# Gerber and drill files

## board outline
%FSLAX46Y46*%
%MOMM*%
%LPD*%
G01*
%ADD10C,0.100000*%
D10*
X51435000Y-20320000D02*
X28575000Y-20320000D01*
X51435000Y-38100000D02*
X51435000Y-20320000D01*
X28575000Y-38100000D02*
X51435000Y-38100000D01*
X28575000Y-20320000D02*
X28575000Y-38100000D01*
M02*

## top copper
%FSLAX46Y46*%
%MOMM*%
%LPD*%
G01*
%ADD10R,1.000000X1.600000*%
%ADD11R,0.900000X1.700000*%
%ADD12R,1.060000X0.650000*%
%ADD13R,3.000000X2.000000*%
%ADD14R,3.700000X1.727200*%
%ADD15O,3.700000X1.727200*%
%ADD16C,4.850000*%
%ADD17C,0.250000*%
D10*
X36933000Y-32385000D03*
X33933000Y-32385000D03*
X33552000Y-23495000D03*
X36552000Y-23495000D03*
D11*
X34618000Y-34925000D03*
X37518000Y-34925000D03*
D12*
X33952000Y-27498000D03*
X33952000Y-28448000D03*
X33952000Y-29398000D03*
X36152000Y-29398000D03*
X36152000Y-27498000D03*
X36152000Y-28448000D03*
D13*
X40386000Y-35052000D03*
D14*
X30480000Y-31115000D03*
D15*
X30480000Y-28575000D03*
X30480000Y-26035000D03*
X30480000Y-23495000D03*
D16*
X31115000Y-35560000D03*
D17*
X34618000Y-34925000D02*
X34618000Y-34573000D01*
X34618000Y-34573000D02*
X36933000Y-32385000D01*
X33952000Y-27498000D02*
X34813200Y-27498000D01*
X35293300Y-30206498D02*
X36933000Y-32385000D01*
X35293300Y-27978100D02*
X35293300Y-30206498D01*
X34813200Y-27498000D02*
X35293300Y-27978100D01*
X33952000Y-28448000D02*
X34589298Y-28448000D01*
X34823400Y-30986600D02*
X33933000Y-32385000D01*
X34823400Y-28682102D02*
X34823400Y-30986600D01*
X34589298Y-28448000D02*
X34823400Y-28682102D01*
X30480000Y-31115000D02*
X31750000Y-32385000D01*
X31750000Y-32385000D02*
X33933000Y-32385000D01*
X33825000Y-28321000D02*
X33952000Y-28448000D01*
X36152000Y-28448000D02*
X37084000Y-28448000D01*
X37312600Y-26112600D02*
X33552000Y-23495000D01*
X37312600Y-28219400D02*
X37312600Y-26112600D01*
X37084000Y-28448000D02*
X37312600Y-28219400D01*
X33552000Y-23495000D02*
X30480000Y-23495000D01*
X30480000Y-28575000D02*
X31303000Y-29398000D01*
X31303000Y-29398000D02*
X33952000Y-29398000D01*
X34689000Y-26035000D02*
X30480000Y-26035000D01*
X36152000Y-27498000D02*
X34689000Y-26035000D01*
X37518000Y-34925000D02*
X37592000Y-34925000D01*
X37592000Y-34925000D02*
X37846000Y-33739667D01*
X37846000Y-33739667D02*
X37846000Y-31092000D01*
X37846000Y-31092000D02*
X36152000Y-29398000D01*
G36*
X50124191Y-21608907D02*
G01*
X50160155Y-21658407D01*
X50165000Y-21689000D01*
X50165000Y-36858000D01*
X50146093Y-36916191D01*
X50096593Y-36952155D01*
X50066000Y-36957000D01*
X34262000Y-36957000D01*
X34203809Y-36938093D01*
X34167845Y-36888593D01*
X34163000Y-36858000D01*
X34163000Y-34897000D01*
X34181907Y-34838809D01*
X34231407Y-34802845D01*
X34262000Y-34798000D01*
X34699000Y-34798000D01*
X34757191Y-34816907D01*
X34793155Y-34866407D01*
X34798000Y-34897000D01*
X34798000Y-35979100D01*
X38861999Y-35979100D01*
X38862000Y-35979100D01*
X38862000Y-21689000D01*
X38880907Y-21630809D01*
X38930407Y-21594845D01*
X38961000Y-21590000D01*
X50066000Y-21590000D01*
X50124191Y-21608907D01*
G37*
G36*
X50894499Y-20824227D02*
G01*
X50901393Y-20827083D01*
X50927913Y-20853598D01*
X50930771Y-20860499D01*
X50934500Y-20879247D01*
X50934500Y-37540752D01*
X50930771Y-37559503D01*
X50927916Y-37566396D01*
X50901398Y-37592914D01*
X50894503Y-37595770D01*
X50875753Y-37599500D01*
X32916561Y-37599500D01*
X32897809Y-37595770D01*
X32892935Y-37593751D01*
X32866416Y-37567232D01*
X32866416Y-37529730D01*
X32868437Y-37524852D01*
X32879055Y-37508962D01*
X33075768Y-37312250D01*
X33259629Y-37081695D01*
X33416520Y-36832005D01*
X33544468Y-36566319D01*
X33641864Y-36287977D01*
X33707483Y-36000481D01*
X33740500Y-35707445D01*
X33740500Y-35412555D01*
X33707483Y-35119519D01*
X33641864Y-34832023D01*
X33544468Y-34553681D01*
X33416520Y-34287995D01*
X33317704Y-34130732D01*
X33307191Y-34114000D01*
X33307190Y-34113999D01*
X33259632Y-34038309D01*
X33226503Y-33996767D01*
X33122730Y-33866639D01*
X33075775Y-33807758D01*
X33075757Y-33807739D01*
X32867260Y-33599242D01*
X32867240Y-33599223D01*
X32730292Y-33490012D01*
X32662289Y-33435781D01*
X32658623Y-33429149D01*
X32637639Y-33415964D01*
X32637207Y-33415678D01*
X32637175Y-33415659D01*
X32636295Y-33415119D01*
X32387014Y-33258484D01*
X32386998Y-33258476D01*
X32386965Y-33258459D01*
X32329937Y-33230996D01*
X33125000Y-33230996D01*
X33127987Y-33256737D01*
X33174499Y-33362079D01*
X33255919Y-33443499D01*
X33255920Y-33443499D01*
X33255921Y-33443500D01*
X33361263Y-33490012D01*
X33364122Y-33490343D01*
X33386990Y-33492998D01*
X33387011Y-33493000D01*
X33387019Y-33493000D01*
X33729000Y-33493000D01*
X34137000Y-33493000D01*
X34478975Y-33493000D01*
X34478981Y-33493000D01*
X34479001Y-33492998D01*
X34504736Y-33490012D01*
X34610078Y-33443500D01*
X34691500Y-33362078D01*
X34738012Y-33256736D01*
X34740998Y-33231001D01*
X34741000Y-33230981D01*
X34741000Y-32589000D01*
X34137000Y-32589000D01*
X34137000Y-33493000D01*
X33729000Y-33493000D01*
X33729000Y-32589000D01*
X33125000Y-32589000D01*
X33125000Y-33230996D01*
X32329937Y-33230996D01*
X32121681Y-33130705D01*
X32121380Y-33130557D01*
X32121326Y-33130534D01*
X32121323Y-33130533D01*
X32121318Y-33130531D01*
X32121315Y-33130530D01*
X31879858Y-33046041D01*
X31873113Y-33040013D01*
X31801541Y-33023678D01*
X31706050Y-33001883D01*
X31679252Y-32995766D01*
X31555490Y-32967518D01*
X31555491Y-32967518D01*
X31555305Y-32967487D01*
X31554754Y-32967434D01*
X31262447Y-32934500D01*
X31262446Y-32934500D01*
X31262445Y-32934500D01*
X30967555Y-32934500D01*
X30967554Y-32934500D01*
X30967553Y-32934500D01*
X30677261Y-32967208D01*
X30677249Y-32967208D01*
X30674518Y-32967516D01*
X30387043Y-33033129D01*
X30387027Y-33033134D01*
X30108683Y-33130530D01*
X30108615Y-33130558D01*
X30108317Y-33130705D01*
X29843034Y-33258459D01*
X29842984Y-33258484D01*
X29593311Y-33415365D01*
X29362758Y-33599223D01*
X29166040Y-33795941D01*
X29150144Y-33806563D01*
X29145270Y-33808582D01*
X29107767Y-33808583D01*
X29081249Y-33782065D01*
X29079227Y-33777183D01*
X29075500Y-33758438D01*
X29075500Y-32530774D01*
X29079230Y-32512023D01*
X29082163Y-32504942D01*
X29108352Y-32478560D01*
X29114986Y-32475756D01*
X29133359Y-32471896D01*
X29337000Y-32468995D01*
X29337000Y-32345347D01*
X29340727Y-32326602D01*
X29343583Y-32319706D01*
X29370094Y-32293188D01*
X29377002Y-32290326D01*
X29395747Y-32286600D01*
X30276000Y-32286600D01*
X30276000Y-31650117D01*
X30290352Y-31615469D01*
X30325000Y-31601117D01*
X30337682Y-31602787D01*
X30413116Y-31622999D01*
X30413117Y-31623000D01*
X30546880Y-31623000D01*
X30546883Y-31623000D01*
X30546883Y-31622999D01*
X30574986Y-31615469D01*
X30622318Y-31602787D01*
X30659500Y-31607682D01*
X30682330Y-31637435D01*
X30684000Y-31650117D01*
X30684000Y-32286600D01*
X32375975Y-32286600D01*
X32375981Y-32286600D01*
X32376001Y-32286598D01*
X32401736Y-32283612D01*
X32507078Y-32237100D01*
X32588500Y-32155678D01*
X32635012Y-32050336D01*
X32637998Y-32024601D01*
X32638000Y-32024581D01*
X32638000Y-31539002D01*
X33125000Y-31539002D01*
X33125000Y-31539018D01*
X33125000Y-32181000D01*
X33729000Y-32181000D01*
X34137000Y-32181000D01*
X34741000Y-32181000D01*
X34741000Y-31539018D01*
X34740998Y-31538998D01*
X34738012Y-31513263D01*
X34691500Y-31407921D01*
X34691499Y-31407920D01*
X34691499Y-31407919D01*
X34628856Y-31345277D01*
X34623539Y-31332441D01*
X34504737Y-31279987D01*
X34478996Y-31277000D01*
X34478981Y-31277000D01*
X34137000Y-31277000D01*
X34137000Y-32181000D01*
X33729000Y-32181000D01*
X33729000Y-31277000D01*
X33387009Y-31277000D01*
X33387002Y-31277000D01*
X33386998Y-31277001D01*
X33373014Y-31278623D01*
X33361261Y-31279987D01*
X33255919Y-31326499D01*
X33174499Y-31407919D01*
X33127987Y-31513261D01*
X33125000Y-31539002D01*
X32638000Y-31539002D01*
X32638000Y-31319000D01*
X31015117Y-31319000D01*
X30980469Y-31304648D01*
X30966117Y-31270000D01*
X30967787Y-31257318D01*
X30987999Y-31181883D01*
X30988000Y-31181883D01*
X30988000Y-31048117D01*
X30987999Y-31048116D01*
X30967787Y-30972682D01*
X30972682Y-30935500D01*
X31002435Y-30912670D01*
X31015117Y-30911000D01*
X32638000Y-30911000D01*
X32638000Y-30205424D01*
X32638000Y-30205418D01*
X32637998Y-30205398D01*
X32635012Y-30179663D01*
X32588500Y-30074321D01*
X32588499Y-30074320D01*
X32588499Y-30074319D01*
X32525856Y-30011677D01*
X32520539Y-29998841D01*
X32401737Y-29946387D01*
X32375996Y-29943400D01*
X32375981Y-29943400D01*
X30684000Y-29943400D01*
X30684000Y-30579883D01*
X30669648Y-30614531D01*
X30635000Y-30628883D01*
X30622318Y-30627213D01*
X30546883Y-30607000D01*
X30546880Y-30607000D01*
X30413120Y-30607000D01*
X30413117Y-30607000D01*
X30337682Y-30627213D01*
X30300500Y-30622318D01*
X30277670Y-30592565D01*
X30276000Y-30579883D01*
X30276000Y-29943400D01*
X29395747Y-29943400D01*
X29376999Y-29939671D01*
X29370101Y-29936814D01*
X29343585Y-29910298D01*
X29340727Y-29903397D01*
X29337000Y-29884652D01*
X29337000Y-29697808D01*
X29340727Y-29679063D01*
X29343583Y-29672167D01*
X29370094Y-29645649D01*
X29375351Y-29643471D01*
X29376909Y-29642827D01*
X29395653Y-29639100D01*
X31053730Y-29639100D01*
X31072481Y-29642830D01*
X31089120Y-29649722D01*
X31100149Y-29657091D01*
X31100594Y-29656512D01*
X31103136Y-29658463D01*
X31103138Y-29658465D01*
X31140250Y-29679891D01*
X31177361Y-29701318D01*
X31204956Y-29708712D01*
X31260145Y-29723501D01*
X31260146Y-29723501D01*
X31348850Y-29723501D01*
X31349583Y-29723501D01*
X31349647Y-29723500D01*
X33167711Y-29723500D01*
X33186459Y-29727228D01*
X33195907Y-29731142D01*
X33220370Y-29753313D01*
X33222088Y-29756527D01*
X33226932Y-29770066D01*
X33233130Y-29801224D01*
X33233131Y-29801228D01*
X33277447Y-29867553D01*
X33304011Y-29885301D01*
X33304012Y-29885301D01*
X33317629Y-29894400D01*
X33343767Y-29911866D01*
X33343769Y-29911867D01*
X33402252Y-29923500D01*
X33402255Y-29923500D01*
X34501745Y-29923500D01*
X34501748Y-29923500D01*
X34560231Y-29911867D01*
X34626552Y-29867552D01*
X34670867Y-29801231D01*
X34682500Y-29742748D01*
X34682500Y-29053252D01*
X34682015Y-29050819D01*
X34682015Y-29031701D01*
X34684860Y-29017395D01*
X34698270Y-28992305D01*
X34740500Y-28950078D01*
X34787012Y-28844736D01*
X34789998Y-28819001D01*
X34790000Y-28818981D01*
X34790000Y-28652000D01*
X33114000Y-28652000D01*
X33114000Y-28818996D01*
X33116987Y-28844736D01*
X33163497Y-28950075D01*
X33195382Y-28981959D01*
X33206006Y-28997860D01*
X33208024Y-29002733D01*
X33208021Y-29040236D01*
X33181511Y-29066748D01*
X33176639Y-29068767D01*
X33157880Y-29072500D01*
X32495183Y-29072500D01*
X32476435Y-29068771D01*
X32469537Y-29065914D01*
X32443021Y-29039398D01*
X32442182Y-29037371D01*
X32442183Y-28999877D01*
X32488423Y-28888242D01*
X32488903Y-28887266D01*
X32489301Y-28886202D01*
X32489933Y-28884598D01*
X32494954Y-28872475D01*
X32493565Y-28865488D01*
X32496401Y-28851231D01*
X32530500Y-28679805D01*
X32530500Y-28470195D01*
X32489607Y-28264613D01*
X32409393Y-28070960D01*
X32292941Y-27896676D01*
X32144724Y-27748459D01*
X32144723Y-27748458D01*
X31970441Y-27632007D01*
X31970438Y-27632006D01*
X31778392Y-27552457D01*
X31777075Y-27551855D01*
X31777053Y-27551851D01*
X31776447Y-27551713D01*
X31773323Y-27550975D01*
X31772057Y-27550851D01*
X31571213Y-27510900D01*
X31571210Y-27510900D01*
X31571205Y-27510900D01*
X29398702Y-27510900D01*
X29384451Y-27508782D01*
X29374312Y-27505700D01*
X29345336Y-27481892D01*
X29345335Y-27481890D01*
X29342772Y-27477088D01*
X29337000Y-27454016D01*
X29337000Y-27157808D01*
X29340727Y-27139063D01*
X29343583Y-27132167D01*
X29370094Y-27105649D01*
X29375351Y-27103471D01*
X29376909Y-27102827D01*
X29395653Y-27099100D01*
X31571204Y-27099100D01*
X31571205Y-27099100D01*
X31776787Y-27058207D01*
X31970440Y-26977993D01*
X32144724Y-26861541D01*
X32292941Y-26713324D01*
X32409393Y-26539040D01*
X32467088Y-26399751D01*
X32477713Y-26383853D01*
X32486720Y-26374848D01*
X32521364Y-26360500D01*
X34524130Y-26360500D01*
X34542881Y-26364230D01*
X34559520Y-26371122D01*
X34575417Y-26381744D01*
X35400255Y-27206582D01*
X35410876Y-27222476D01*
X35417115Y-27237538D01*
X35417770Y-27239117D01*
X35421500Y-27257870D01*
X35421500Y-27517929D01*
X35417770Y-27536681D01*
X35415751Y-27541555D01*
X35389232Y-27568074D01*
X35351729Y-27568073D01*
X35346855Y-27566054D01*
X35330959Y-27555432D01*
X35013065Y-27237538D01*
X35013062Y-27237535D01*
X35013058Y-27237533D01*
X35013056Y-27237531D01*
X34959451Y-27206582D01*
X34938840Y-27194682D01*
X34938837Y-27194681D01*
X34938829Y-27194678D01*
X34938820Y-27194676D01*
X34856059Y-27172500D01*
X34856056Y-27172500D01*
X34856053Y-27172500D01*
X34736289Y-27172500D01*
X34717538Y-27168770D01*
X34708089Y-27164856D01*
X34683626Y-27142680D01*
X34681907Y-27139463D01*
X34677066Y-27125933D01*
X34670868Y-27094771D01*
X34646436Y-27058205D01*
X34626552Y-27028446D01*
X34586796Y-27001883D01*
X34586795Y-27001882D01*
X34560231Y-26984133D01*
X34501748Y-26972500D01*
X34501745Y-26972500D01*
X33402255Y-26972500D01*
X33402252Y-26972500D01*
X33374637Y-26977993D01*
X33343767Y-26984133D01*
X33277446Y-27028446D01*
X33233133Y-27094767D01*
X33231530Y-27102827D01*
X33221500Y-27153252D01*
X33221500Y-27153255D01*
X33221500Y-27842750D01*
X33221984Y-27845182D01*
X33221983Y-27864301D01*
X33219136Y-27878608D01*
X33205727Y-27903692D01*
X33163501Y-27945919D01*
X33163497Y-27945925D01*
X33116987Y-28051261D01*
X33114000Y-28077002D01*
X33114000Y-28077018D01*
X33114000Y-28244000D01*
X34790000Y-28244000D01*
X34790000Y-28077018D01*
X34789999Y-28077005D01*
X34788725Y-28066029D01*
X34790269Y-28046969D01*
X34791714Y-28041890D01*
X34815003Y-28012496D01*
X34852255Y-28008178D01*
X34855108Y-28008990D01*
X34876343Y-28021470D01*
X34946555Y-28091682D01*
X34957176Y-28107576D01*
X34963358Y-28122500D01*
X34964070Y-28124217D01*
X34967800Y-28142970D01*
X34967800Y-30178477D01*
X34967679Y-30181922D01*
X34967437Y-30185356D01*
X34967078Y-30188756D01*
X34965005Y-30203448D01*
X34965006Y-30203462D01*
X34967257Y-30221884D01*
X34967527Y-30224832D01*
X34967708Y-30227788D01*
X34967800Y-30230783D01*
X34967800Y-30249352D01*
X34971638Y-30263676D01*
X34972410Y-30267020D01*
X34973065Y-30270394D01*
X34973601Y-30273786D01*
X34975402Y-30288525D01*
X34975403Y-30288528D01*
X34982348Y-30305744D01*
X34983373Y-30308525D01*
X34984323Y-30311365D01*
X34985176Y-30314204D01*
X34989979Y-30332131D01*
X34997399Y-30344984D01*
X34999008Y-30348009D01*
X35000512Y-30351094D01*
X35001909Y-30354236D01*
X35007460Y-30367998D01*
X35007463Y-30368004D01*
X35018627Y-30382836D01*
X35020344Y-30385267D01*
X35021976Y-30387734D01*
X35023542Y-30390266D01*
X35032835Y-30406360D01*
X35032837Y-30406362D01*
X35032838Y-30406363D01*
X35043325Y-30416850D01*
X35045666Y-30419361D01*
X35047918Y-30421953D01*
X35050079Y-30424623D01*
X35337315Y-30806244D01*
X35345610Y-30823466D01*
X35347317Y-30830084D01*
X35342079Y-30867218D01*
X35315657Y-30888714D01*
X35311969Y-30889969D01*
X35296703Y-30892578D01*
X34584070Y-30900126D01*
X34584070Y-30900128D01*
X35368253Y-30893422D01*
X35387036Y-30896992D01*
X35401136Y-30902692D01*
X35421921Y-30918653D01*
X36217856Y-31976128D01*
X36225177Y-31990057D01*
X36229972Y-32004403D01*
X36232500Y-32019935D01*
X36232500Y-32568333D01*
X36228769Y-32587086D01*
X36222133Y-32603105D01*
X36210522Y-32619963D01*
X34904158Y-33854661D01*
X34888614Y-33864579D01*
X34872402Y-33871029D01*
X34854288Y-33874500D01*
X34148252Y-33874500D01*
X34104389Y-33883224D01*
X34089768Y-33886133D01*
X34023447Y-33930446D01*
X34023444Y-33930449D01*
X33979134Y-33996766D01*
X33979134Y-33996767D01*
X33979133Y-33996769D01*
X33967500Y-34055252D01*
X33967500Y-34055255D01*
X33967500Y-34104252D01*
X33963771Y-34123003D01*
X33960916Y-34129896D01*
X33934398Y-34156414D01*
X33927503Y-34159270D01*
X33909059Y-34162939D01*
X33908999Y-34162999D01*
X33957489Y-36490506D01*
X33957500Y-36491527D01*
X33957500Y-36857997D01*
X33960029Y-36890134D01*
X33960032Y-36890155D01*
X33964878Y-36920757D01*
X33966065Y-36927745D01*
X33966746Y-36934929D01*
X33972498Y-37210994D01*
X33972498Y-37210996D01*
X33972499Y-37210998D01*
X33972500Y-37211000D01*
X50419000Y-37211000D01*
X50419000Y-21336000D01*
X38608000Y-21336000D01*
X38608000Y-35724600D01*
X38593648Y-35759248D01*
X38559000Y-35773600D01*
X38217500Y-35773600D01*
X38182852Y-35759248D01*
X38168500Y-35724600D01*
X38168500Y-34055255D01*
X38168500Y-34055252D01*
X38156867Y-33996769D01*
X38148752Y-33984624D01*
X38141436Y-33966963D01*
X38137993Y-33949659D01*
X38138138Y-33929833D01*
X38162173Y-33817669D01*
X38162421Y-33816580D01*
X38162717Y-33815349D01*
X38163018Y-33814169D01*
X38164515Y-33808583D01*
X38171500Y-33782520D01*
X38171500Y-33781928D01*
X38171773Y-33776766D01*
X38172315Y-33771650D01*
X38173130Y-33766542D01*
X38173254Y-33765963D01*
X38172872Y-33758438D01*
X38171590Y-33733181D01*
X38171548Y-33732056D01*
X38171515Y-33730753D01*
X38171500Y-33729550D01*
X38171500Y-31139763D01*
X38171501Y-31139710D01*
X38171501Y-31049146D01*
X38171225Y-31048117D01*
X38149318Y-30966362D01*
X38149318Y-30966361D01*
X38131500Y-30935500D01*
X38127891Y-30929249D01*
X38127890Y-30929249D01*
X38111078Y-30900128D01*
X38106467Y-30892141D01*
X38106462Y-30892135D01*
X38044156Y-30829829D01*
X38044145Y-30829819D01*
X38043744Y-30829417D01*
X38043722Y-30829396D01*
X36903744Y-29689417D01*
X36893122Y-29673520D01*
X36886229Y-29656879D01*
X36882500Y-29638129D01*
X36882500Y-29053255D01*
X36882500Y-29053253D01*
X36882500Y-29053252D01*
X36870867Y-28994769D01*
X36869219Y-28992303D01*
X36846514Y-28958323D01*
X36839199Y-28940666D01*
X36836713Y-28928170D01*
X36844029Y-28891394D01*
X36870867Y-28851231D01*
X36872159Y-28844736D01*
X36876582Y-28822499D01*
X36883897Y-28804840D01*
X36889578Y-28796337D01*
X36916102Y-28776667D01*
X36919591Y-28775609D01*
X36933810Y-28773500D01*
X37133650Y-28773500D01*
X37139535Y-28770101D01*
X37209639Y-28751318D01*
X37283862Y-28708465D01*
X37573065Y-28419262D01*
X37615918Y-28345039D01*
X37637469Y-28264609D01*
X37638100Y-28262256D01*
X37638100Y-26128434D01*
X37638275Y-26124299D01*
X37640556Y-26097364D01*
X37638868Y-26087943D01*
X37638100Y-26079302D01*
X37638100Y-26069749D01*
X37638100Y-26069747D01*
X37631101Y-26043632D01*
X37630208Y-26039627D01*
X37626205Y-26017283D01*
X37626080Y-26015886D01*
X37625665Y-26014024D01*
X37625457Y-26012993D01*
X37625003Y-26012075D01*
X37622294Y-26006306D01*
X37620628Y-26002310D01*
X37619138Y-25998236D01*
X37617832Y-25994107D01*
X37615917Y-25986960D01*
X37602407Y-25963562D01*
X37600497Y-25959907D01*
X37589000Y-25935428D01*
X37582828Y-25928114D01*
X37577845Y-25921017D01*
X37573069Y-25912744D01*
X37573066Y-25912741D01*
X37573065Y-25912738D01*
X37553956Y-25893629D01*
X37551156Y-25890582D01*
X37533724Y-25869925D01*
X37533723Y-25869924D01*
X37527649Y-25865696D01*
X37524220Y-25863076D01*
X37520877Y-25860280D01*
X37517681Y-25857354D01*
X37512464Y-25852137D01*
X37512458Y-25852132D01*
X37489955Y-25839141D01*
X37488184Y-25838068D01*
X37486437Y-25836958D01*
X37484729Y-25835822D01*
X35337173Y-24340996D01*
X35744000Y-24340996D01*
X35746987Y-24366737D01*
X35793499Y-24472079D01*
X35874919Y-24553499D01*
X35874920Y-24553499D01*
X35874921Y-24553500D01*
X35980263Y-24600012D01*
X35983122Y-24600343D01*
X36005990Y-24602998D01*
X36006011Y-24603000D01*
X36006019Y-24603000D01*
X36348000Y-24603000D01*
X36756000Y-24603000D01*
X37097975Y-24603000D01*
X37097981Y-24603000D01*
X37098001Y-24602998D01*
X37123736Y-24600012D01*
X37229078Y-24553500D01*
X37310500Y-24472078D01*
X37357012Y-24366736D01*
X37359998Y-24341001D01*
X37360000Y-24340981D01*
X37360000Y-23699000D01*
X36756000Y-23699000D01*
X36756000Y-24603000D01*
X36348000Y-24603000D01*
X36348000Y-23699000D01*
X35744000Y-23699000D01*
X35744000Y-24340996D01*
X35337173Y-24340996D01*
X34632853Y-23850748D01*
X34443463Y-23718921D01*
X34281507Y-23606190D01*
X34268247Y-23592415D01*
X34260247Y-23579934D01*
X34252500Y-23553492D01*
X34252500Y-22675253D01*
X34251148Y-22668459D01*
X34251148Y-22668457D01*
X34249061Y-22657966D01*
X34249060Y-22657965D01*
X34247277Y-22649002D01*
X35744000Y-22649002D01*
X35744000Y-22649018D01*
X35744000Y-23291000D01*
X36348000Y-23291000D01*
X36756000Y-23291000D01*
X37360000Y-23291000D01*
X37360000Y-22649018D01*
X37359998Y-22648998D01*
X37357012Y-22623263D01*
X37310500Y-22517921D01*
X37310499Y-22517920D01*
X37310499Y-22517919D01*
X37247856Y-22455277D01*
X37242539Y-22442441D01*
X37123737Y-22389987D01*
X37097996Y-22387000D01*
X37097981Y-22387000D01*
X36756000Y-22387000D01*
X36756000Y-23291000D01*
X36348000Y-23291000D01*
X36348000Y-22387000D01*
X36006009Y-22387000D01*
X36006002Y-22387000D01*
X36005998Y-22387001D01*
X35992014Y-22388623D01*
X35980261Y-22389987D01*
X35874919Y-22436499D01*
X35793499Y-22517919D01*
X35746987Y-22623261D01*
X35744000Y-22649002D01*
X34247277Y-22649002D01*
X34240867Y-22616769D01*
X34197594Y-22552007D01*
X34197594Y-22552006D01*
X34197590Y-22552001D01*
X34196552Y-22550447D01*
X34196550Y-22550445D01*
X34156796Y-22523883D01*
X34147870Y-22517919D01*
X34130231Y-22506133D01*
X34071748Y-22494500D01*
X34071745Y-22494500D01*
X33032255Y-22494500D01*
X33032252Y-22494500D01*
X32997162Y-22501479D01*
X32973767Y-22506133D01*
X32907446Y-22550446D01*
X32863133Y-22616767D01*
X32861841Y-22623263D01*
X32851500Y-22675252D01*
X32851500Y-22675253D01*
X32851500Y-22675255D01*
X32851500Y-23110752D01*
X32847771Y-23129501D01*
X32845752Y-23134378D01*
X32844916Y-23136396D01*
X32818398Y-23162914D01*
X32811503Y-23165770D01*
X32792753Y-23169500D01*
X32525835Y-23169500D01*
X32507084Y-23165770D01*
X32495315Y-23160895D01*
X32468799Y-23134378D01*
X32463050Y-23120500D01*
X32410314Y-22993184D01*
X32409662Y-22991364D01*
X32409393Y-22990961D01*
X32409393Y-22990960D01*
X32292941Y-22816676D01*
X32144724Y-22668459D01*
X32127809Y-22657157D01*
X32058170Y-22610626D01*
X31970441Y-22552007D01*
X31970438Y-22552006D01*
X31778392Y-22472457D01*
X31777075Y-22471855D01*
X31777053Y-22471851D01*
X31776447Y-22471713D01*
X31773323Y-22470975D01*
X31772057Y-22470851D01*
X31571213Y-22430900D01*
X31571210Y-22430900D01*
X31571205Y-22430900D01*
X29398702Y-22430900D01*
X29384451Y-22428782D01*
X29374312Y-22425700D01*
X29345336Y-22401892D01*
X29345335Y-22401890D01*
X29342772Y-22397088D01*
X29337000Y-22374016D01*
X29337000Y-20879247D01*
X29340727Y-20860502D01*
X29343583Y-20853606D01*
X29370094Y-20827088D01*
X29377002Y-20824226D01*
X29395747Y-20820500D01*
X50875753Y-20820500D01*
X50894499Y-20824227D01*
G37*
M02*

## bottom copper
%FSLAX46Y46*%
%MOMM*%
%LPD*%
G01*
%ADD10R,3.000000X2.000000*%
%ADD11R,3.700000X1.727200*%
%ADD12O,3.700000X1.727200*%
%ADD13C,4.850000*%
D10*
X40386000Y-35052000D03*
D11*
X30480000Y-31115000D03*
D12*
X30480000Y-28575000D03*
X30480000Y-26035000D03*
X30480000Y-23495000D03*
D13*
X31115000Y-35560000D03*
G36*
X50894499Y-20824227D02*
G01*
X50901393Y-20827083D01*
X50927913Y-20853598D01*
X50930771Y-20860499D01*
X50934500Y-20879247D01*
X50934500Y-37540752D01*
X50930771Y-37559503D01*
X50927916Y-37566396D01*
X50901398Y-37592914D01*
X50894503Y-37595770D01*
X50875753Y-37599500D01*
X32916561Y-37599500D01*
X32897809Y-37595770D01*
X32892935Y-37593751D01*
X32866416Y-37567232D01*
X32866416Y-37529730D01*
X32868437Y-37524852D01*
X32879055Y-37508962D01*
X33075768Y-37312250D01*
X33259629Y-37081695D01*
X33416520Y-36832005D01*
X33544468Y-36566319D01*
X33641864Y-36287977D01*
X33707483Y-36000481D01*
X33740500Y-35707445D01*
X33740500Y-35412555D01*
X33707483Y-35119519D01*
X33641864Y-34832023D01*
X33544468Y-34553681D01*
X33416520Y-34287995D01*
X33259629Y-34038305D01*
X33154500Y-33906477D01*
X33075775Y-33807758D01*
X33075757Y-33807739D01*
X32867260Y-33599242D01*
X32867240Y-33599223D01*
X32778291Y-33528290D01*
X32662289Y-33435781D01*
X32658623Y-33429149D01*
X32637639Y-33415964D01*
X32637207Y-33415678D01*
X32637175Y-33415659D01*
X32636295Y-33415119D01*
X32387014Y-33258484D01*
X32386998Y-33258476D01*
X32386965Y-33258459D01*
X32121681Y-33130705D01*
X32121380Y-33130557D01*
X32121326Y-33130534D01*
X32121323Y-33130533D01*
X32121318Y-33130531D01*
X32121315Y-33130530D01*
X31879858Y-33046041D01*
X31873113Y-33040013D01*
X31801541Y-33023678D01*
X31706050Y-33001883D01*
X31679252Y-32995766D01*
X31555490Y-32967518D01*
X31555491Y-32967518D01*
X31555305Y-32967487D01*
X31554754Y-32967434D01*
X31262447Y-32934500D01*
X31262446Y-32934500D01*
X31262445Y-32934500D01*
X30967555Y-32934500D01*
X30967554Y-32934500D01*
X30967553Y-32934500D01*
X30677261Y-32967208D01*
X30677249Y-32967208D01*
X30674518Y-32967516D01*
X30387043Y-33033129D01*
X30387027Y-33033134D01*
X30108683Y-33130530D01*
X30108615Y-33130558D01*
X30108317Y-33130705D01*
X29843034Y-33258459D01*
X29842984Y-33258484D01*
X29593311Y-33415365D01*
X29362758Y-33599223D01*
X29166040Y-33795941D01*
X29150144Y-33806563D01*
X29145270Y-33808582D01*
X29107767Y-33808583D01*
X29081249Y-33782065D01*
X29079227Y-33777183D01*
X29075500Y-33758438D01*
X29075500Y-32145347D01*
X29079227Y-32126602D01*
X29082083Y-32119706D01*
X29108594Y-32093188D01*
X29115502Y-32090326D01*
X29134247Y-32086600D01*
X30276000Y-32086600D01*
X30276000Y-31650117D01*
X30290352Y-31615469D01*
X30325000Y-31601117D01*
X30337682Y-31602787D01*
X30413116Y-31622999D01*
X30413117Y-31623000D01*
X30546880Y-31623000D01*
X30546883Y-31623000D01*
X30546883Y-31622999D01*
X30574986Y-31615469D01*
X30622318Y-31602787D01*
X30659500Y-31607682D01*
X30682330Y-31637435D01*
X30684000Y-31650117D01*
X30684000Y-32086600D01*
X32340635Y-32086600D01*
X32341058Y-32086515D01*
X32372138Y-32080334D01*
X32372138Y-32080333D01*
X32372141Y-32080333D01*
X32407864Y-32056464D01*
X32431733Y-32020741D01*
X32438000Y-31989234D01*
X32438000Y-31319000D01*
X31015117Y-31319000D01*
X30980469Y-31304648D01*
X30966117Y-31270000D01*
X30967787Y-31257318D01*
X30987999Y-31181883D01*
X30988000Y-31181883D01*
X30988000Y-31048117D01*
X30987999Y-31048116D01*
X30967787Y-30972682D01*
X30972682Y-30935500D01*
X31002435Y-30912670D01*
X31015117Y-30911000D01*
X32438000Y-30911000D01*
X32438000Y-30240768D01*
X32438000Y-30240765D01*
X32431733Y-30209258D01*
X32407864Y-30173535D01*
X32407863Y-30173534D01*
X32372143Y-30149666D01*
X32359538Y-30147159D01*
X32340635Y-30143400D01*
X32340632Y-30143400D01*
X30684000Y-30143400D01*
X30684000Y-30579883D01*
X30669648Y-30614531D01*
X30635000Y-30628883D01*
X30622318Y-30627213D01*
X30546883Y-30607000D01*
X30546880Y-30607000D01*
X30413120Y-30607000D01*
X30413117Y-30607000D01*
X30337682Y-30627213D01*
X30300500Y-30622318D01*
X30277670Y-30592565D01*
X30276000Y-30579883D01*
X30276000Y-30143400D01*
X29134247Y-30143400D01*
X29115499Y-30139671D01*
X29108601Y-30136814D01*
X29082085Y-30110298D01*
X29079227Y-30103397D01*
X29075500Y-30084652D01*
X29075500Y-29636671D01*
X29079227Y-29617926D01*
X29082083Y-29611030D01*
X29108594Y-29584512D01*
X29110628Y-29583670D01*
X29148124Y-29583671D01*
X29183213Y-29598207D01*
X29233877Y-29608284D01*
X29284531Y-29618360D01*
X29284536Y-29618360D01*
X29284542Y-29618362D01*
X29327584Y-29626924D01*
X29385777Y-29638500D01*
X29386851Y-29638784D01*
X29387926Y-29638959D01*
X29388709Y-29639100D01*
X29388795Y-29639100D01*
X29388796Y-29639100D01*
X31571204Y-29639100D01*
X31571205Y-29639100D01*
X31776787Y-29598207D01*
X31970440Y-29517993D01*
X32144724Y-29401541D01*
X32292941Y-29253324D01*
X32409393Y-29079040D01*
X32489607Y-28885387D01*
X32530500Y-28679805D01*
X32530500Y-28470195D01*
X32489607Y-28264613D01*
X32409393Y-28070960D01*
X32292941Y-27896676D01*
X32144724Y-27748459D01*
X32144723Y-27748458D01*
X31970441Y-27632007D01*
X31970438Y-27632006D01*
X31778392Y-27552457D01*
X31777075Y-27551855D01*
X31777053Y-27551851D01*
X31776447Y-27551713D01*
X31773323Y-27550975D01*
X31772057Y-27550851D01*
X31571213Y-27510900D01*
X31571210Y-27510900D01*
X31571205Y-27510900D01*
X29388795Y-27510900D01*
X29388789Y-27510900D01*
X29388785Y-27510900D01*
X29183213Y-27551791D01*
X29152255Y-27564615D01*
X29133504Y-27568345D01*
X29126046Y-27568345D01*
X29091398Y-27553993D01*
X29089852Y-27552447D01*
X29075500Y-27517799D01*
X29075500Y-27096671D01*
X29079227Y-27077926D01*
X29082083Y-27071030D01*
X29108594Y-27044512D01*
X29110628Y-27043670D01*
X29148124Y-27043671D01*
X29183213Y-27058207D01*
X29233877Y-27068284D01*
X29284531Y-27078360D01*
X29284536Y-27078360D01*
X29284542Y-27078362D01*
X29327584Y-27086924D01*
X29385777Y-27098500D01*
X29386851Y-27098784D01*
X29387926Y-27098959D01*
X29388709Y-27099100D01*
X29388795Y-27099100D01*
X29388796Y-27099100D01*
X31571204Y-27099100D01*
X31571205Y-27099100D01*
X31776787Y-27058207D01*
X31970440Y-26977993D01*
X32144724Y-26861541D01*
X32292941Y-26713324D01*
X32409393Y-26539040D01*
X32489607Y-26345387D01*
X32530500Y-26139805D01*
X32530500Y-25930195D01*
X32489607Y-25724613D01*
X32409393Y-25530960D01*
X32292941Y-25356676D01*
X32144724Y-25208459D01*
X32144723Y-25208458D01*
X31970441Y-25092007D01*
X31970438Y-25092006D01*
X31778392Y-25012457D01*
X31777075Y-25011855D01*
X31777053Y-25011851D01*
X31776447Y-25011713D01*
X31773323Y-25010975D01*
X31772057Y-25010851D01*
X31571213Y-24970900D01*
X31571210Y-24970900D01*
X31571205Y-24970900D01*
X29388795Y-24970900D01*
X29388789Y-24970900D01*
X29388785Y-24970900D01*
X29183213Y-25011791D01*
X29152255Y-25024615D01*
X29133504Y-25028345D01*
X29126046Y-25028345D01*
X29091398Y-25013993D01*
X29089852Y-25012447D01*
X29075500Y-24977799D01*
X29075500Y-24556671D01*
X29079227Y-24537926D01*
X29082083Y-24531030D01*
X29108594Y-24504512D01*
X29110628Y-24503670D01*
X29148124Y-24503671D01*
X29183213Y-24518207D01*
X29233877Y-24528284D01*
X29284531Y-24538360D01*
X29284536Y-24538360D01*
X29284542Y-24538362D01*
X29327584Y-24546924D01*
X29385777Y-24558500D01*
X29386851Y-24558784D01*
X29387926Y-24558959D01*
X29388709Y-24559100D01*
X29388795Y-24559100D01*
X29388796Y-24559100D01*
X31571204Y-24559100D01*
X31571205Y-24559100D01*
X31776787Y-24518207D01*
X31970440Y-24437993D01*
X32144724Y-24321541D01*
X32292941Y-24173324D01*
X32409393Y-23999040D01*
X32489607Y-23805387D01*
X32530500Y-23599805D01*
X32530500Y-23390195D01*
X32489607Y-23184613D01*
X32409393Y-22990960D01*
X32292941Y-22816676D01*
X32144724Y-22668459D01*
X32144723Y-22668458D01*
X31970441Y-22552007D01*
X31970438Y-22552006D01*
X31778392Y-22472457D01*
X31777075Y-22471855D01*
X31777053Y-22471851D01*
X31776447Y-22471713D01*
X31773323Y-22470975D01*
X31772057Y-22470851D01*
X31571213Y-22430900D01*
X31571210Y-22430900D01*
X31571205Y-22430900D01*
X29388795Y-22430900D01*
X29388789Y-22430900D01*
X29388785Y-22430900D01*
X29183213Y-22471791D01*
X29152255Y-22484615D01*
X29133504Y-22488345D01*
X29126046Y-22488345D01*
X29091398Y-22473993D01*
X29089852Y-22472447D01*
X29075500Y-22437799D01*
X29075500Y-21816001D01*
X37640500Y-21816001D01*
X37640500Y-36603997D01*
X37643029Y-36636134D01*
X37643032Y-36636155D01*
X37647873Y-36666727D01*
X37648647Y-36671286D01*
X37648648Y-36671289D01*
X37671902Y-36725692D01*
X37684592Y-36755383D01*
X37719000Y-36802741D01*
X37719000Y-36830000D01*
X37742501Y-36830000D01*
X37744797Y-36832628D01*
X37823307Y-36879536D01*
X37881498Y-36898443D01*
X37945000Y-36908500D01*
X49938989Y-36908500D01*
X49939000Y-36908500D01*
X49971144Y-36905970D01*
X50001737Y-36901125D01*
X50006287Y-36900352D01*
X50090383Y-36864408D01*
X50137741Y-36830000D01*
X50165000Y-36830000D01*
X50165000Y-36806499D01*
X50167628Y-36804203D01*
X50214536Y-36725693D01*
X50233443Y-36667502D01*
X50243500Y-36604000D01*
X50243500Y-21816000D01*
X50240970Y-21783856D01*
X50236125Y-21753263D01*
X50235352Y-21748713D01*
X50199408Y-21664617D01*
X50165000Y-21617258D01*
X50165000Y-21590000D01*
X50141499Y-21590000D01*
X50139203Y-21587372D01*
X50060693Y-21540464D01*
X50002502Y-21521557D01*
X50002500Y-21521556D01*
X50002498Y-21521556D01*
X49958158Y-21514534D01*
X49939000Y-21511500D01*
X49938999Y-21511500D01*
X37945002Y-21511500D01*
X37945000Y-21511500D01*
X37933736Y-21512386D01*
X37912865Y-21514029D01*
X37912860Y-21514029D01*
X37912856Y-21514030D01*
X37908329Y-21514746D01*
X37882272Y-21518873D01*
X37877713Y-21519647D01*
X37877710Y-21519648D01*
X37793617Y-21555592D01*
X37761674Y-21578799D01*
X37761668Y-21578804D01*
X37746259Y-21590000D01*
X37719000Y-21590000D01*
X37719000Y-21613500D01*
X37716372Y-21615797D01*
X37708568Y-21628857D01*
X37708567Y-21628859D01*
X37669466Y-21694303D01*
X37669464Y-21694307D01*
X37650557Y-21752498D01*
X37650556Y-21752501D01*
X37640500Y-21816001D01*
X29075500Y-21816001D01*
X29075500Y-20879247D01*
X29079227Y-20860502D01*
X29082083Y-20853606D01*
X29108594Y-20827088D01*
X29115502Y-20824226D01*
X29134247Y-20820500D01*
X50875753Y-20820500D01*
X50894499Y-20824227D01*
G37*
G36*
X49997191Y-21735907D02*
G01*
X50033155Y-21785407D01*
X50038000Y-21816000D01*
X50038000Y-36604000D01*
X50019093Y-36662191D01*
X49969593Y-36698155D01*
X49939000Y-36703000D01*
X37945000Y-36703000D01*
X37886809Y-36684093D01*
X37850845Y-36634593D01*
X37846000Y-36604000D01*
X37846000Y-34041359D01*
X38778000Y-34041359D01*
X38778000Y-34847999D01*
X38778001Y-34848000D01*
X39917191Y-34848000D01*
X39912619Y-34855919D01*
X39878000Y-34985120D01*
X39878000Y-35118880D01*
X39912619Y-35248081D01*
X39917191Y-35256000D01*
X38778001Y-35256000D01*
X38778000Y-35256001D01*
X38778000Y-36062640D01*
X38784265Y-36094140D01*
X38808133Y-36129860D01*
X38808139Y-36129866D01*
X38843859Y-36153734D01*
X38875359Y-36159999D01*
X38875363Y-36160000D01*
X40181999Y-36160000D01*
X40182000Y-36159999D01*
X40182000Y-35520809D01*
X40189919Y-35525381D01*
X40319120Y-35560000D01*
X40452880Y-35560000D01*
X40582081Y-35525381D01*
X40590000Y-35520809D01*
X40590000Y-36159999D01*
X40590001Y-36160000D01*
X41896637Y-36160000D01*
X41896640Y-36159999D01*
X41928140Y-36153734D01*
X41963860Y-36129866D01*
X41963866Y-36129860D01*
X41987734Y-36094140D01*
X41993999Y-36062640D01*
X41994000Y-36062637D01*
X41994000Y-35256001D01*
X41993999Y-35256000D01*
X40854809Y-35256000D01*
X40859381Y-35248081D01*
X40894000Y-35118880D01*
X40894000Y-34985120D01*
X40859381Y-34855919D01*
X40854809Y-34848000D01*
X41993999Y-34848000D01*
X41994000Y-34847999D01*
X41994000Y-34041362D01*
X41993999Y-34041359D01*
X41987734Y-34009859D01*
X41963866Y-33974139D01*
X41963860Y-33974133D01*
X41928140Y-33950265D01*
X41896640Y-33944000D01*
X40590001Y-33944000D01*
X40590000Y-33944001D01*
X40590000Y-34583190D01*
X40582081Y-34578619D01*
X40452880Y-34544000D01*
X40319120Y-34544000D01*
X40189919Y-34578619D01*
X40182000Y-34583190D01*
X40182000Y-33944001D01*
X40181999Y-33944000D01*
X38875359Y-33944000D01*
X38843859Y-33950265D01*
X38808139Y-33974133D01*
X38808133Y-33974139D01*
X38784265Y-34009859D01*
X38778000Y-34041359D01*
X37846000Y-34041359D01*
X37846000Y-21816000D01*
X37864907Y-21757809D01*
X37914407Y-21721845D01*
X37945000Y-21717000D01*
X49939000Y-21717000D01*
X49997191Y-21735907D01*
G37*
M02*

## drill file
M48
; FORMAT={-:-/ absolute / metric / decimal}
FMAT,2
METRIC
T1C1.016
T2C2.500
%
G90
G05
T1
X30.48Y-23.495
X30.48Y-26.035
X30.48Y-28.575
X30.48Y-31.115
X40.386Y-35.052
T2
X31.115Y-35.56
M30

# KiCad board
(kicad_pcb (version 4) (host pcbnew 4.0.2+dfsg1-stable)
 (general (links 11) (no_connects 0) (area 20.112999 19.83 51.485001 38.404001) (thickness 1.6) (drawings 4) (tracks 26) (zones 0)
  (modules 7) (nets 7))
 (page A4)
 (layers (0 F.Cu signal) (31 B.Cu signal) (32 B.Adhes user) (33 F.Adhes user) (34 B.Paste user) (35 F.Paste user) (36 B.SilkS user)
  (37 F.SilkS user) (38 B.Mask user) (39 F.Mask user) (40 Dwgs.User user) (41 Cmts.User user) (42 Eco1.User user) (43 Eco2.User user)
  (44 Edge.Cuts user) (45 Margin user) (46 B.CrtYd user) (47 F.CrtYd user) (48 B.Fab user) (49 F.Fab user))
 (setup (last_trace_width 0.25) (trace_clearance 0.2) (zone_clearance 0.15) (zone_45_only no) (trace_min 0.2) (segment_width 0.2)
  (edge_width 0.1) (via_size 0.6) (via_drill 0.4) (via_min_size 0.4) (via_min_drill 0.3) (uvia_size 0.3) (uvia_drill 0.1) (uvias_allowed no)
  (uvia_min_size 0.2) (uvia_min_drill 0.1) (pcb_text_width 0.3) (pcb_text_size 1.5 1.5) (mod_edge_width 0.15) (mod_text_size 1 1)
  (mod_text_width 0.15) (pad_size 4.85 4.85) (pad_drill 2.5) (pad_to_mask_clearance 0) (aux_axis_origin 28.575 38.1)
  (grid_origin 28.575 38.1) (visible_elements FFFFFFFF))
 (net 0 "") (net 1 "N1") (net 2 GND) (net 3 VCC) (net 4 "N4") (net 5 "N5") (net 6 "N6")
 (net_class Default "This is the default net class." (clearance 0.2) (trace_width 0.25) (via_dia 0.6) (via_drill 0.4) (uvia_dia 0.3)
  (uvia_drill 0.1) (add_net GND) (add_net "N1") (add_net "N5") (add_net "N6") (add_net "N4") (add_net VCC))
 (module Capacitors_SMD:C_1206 (layer F.Cu) (at 35.433 32.385 180)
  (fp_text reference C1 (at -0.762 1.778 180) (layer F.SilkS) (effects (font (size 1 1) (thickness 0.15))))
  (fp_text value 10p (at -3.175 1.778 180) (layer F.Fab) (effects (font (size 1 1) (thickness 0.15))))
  (pad 1 smd rect (at -1.5 0 180) (size 1 1.6) (layers F.Cu F.Paste F.Mask) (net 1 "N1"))
  (pad 2 smd rect (at 1.5 0 180) (size 1 1.6) (layers F.Cu F.Paste F.Mask) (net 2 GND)))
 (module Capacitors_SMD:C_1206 (layer F.Cu) (at 35.052 23.495)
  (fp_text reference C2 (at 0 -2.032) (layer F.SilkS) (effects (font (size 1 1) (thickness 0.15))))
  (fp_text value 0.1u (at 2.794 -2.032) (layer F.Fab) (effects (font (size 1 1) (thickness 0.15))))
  (pad 1 smd rect (at -1.5 0) (size 1 1.6) (layers F.Cu F.Paste F.Mask) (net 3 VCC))
  (pad 2 smd rect (at 1.5 0) (size 1 1.6) (layers F.Cu F.Paste F.Mask) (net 2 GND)))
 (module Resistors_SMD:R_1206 (layer F.Cu) (at 36.068 34.925)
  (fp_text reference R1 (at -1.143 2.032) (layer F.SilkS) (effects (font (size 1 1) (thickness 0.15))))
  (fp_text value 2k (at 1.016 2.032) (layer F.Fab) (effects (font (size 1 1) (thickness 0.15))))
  (pad 1 smd rect (at -1.45 0) (size 0.9 1.7) (layers F.Cu F.Paste F.Mask) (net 1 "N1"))
  (pad 2 smd rect (at 1.45 0) (size 0.9 1.7) (layers F.Cu F.Paste F.Mask) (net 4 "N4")))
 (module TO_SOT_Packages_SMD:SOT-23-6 (layer F.Cu) (at 35.052 28.448)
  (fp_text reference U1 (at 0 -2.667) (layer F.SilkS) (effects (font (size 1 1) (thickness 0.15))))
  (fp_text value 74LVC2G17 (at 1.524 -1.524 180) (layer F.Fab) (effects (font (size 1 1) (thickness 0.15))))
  (pad 1 smd rect (at -1.1 -0.95) (size 1.06 0.65) (layers F.Cu F.Paste F.Mask) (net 1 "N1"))
  (pad 2 smd rect (at -1.1 0) (size 1.06 0.65) (layers F.Cu F.Paste F.Mask) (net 2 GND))
  (pad 3 smd rect (at -1.1 0.95) (size 1.06 0.65) (layers F.Cu F.Paste F.Mask) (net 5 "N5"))
  (pad 4 smd rect (at 1.1 0.95) (size 1.06 0.65) (layers F.Cu F.Paste F.Mask) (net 4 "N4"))
  (pad 6 smd rect (at 1.1 -0.95) (size 1.06 0.65) (layers F.Cu F.Paste F.Mask) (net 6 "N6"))
  (pad 5 smd rect (at 1.1 0) (size 1.06 0.65) (layers F.Cu F.Paste F.Mask) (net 3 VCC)))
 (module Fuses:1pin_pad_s (layer F.Cu) (at 40.386 35.052)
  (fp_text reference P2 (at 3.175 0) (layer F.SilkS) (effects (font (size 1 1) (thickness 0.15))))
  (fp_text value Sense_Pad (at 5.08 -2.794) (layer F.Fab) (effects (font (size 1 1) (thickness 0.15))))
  (pad 1 thru_hole rect (at 0 0) (size 3 2) (drill 1.016) (layers *.Cu *.Mask F.SilkS) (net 1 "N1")))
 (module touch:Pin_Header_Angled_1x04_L (layer F.Cu) (at 30.48 31.115 180)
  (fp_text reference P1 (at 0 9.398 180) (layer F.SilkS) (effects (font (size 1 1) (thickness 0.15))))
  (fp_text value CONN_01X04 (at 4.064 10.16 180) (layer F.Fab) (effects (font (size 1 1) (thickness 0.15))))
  (pad 1 thru_hole rect (at 0 0 180) (size 3.7 1.7272) (drill 1.016) (layers *.Cu *.Mask F.SilkS) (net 2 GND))
  (pad 2 thru_hole oval (at 0 2.54 180) (size 3.7 1.7272) (drill 1.016) (layers *.Cu *.Mask F.SilkS) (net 5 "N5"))
  (pad 3 thru_hole oval (at 0 5.08 180) (size 3.7 1.7272) (drill 1.016) (layers *.Cu *.Mask F.SilkS) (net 6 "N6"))
  (pad 4 thru_hole oval (at 0 7.62 180) (size 3.7 1.7272) (drill 1.016) (layers *.Cu *.Mask F.SilkS) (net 3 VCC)))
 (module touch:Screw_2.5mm (layer F.Cu) (at 31.115 35.56)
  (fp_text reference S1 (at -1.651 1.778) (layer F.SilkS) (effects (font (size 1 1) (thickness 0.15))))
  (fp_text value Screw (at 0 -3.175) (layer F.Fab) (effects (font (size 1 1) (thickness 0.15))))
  (pad 1 thru_hole circle (at 0 0) (size 4.85 4.85) (drill 2.5) (layers *.Cu *.Mask F.SilkS)))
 (gr_line (start 51.435 20.32) (end 28.575 20.32) (angle 90) (layer Edge.Cuts) (width 0.1))
 (gr_line (start 51.435 38.1) (end 51.435 20.32) (angle 90) (layer Edge.Cuts) (width 0.1))
 (gr_line (start 28.575 38.1) (end 51.435 38.1) (angle 90) (layer Edge.Cuts) (width 0.1))
 (gr_line (start 28.575 20.32) (end 28.575 38.1) (angle 90) (layer Edge.Cuts) (width 0.1))
 (segment (start 34.618 34.925) (end 34.618 34.573) (width 0.25) (layer F.Cu) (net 1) (status 30))
 (segment (start 34.618 34.573) (end 36.933 32.385) (width 0.25) (layer F.Cu) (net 1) (status 10))
 (segment (start 33.952 27.498) (end 34.8132 27.498) (width 0.25) (layer F.Cu) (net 1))
 (segment (start 35.2933 30.206498) (end 36.933 32.385) (width 0.25) (layer F.Cu) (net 1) (status 20))
 (segment (start 35.2933 27.9781) (end 35.2933 30.206498) (width 0.25) (layer F.Cu) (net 1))
 (segment (start 34.8132 27.498) (end 35.2933 27.9781) (width 0.25) (layer F.Cu) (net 1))
 (segment (start 33.952 28.448) (end 34.589298 28.448) (width 0.25) (layer F.Cu) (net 2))
 (segment (start 34.8234 30.9866) (end 33.933 32.385) (width 0.25) (layer F.Cu) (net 2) (status 20))
 (segment (start 34.8234 28.682102) (end 34.8234 30.9866) (width 0.25) (layer F.Cu) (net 2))
 (segment (start 34.589298 28.448) (end 34.8234 28.682102) (width 0.25) (layer F.Cu) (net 2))
 (segment (start 30.48 31.115) (end 31.75 32.385) (width 0.25) (layer F.Cu) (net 2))
 (segment (start 31.75 32.385) (end 33.933 32.385) (width 0.25) (layer F.Cu) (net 2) (status 20))
 (segment (start 33.825 28.321) (end 33.952 28.448) (width 0.25) (layer F.Cu) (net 2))
 (segment (start 36.152 28.448) (end 37.084 28.448) (width 0.25) (layer F.Cu) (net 3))
 (segment (start 37.3126 26.1126) (end 33.552 23.495) (width 0.25) (layer F.Cu) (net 3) (status 20))
 (segment (start 37.3126 28.2194) (end 37.3126 26.1126) (width 0.25) (layer F.Cu) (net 3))
 (segment (start 37.084 28.448) (end 37.3126 28.2194) (width 0.25) (layer F.Cu) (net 3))
 (segment (start 33.552 23.495) (end 30.48 23.495) (width 0.25) (layer F.Cu) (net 3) (status 10))
 (segment (start 30.48 28.575) (end 31.303 29.398) (width 0.25) (layer F.Cu) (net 5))
 (segment (start 31.303 29.398) (end 33.952 29.398) (width 0.25) (layer F.Cu) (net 5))
 (segment (start 34.689 26.035) (end 30.48 26.035) (width 0.25) (layer F.Cu) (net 6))
 (segment (start 36.152 27.498) (end 34.689 26.035) (width 0.25) (layer F.Cu) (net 6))
 (segment (start 37.518 34.925) (end 37.592 34.925) (width 0.25) (layer F.Cu) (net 4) (status 30))
 (segment (start 37.592 34.925) (end 37.846 33.739667) (width 0.25) (layer F.Cu) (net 4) (status 10))
 (segment (start 37.846 33.739667) (end 37.846 31.092) (width 0.25) (layer F.Cu) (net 4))
 (segment (start 37.846 31.092) (end 36.152 29.398) (width 0.25) (layer F.Cu) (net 4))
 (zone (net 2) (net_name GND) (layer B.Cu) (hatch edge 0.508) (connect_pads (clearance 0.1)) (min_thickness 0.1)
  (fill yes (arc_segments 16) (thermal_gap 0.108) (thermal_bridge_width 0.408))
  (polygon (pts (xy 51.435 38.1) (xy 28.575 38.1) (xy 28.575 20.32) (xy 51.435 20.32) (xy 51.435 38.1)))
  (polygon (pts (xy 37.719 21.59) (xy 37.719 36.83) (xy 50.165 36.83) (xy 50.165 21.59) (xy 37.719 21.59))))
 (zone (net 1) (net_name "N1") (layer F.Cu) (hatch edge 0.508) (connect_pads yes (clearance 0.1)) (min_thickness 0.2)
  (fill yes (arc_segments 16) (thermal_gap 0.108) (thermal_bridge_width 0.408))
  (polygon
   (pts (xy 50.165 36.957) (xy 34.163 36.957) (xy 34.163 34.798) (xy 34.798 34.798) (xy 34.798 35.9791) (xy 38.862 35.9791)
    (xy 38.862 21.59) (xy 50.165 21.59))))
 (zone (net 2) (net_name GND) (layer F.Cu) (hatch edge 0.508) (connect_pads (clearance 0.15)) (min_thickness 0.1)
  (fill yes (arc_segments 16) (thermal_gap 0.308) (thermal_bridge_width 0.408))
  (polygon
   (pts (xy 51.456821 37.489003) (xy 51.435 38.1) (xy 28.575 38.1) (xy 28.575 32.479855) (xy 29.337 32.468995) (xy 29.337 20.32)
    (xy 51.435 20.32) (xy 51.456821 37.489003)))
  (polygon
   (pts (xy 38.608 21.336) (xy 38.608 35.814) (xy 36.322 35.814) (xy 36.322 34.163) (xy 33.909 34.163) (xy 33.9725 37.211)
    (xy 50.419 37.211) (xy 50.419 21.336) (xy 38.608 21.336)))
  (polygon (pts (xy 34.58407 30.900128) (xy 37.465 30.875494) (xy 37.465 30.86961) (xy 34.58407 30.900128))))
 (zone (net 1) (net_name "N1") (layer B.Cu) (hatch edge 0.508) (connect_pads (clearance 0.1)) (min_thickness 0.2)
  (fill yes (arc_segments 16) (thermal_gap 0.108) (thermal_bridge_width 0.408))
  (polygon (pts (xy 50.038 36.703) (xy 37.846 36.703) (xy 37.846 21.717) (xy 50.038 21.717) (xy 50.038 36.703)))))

